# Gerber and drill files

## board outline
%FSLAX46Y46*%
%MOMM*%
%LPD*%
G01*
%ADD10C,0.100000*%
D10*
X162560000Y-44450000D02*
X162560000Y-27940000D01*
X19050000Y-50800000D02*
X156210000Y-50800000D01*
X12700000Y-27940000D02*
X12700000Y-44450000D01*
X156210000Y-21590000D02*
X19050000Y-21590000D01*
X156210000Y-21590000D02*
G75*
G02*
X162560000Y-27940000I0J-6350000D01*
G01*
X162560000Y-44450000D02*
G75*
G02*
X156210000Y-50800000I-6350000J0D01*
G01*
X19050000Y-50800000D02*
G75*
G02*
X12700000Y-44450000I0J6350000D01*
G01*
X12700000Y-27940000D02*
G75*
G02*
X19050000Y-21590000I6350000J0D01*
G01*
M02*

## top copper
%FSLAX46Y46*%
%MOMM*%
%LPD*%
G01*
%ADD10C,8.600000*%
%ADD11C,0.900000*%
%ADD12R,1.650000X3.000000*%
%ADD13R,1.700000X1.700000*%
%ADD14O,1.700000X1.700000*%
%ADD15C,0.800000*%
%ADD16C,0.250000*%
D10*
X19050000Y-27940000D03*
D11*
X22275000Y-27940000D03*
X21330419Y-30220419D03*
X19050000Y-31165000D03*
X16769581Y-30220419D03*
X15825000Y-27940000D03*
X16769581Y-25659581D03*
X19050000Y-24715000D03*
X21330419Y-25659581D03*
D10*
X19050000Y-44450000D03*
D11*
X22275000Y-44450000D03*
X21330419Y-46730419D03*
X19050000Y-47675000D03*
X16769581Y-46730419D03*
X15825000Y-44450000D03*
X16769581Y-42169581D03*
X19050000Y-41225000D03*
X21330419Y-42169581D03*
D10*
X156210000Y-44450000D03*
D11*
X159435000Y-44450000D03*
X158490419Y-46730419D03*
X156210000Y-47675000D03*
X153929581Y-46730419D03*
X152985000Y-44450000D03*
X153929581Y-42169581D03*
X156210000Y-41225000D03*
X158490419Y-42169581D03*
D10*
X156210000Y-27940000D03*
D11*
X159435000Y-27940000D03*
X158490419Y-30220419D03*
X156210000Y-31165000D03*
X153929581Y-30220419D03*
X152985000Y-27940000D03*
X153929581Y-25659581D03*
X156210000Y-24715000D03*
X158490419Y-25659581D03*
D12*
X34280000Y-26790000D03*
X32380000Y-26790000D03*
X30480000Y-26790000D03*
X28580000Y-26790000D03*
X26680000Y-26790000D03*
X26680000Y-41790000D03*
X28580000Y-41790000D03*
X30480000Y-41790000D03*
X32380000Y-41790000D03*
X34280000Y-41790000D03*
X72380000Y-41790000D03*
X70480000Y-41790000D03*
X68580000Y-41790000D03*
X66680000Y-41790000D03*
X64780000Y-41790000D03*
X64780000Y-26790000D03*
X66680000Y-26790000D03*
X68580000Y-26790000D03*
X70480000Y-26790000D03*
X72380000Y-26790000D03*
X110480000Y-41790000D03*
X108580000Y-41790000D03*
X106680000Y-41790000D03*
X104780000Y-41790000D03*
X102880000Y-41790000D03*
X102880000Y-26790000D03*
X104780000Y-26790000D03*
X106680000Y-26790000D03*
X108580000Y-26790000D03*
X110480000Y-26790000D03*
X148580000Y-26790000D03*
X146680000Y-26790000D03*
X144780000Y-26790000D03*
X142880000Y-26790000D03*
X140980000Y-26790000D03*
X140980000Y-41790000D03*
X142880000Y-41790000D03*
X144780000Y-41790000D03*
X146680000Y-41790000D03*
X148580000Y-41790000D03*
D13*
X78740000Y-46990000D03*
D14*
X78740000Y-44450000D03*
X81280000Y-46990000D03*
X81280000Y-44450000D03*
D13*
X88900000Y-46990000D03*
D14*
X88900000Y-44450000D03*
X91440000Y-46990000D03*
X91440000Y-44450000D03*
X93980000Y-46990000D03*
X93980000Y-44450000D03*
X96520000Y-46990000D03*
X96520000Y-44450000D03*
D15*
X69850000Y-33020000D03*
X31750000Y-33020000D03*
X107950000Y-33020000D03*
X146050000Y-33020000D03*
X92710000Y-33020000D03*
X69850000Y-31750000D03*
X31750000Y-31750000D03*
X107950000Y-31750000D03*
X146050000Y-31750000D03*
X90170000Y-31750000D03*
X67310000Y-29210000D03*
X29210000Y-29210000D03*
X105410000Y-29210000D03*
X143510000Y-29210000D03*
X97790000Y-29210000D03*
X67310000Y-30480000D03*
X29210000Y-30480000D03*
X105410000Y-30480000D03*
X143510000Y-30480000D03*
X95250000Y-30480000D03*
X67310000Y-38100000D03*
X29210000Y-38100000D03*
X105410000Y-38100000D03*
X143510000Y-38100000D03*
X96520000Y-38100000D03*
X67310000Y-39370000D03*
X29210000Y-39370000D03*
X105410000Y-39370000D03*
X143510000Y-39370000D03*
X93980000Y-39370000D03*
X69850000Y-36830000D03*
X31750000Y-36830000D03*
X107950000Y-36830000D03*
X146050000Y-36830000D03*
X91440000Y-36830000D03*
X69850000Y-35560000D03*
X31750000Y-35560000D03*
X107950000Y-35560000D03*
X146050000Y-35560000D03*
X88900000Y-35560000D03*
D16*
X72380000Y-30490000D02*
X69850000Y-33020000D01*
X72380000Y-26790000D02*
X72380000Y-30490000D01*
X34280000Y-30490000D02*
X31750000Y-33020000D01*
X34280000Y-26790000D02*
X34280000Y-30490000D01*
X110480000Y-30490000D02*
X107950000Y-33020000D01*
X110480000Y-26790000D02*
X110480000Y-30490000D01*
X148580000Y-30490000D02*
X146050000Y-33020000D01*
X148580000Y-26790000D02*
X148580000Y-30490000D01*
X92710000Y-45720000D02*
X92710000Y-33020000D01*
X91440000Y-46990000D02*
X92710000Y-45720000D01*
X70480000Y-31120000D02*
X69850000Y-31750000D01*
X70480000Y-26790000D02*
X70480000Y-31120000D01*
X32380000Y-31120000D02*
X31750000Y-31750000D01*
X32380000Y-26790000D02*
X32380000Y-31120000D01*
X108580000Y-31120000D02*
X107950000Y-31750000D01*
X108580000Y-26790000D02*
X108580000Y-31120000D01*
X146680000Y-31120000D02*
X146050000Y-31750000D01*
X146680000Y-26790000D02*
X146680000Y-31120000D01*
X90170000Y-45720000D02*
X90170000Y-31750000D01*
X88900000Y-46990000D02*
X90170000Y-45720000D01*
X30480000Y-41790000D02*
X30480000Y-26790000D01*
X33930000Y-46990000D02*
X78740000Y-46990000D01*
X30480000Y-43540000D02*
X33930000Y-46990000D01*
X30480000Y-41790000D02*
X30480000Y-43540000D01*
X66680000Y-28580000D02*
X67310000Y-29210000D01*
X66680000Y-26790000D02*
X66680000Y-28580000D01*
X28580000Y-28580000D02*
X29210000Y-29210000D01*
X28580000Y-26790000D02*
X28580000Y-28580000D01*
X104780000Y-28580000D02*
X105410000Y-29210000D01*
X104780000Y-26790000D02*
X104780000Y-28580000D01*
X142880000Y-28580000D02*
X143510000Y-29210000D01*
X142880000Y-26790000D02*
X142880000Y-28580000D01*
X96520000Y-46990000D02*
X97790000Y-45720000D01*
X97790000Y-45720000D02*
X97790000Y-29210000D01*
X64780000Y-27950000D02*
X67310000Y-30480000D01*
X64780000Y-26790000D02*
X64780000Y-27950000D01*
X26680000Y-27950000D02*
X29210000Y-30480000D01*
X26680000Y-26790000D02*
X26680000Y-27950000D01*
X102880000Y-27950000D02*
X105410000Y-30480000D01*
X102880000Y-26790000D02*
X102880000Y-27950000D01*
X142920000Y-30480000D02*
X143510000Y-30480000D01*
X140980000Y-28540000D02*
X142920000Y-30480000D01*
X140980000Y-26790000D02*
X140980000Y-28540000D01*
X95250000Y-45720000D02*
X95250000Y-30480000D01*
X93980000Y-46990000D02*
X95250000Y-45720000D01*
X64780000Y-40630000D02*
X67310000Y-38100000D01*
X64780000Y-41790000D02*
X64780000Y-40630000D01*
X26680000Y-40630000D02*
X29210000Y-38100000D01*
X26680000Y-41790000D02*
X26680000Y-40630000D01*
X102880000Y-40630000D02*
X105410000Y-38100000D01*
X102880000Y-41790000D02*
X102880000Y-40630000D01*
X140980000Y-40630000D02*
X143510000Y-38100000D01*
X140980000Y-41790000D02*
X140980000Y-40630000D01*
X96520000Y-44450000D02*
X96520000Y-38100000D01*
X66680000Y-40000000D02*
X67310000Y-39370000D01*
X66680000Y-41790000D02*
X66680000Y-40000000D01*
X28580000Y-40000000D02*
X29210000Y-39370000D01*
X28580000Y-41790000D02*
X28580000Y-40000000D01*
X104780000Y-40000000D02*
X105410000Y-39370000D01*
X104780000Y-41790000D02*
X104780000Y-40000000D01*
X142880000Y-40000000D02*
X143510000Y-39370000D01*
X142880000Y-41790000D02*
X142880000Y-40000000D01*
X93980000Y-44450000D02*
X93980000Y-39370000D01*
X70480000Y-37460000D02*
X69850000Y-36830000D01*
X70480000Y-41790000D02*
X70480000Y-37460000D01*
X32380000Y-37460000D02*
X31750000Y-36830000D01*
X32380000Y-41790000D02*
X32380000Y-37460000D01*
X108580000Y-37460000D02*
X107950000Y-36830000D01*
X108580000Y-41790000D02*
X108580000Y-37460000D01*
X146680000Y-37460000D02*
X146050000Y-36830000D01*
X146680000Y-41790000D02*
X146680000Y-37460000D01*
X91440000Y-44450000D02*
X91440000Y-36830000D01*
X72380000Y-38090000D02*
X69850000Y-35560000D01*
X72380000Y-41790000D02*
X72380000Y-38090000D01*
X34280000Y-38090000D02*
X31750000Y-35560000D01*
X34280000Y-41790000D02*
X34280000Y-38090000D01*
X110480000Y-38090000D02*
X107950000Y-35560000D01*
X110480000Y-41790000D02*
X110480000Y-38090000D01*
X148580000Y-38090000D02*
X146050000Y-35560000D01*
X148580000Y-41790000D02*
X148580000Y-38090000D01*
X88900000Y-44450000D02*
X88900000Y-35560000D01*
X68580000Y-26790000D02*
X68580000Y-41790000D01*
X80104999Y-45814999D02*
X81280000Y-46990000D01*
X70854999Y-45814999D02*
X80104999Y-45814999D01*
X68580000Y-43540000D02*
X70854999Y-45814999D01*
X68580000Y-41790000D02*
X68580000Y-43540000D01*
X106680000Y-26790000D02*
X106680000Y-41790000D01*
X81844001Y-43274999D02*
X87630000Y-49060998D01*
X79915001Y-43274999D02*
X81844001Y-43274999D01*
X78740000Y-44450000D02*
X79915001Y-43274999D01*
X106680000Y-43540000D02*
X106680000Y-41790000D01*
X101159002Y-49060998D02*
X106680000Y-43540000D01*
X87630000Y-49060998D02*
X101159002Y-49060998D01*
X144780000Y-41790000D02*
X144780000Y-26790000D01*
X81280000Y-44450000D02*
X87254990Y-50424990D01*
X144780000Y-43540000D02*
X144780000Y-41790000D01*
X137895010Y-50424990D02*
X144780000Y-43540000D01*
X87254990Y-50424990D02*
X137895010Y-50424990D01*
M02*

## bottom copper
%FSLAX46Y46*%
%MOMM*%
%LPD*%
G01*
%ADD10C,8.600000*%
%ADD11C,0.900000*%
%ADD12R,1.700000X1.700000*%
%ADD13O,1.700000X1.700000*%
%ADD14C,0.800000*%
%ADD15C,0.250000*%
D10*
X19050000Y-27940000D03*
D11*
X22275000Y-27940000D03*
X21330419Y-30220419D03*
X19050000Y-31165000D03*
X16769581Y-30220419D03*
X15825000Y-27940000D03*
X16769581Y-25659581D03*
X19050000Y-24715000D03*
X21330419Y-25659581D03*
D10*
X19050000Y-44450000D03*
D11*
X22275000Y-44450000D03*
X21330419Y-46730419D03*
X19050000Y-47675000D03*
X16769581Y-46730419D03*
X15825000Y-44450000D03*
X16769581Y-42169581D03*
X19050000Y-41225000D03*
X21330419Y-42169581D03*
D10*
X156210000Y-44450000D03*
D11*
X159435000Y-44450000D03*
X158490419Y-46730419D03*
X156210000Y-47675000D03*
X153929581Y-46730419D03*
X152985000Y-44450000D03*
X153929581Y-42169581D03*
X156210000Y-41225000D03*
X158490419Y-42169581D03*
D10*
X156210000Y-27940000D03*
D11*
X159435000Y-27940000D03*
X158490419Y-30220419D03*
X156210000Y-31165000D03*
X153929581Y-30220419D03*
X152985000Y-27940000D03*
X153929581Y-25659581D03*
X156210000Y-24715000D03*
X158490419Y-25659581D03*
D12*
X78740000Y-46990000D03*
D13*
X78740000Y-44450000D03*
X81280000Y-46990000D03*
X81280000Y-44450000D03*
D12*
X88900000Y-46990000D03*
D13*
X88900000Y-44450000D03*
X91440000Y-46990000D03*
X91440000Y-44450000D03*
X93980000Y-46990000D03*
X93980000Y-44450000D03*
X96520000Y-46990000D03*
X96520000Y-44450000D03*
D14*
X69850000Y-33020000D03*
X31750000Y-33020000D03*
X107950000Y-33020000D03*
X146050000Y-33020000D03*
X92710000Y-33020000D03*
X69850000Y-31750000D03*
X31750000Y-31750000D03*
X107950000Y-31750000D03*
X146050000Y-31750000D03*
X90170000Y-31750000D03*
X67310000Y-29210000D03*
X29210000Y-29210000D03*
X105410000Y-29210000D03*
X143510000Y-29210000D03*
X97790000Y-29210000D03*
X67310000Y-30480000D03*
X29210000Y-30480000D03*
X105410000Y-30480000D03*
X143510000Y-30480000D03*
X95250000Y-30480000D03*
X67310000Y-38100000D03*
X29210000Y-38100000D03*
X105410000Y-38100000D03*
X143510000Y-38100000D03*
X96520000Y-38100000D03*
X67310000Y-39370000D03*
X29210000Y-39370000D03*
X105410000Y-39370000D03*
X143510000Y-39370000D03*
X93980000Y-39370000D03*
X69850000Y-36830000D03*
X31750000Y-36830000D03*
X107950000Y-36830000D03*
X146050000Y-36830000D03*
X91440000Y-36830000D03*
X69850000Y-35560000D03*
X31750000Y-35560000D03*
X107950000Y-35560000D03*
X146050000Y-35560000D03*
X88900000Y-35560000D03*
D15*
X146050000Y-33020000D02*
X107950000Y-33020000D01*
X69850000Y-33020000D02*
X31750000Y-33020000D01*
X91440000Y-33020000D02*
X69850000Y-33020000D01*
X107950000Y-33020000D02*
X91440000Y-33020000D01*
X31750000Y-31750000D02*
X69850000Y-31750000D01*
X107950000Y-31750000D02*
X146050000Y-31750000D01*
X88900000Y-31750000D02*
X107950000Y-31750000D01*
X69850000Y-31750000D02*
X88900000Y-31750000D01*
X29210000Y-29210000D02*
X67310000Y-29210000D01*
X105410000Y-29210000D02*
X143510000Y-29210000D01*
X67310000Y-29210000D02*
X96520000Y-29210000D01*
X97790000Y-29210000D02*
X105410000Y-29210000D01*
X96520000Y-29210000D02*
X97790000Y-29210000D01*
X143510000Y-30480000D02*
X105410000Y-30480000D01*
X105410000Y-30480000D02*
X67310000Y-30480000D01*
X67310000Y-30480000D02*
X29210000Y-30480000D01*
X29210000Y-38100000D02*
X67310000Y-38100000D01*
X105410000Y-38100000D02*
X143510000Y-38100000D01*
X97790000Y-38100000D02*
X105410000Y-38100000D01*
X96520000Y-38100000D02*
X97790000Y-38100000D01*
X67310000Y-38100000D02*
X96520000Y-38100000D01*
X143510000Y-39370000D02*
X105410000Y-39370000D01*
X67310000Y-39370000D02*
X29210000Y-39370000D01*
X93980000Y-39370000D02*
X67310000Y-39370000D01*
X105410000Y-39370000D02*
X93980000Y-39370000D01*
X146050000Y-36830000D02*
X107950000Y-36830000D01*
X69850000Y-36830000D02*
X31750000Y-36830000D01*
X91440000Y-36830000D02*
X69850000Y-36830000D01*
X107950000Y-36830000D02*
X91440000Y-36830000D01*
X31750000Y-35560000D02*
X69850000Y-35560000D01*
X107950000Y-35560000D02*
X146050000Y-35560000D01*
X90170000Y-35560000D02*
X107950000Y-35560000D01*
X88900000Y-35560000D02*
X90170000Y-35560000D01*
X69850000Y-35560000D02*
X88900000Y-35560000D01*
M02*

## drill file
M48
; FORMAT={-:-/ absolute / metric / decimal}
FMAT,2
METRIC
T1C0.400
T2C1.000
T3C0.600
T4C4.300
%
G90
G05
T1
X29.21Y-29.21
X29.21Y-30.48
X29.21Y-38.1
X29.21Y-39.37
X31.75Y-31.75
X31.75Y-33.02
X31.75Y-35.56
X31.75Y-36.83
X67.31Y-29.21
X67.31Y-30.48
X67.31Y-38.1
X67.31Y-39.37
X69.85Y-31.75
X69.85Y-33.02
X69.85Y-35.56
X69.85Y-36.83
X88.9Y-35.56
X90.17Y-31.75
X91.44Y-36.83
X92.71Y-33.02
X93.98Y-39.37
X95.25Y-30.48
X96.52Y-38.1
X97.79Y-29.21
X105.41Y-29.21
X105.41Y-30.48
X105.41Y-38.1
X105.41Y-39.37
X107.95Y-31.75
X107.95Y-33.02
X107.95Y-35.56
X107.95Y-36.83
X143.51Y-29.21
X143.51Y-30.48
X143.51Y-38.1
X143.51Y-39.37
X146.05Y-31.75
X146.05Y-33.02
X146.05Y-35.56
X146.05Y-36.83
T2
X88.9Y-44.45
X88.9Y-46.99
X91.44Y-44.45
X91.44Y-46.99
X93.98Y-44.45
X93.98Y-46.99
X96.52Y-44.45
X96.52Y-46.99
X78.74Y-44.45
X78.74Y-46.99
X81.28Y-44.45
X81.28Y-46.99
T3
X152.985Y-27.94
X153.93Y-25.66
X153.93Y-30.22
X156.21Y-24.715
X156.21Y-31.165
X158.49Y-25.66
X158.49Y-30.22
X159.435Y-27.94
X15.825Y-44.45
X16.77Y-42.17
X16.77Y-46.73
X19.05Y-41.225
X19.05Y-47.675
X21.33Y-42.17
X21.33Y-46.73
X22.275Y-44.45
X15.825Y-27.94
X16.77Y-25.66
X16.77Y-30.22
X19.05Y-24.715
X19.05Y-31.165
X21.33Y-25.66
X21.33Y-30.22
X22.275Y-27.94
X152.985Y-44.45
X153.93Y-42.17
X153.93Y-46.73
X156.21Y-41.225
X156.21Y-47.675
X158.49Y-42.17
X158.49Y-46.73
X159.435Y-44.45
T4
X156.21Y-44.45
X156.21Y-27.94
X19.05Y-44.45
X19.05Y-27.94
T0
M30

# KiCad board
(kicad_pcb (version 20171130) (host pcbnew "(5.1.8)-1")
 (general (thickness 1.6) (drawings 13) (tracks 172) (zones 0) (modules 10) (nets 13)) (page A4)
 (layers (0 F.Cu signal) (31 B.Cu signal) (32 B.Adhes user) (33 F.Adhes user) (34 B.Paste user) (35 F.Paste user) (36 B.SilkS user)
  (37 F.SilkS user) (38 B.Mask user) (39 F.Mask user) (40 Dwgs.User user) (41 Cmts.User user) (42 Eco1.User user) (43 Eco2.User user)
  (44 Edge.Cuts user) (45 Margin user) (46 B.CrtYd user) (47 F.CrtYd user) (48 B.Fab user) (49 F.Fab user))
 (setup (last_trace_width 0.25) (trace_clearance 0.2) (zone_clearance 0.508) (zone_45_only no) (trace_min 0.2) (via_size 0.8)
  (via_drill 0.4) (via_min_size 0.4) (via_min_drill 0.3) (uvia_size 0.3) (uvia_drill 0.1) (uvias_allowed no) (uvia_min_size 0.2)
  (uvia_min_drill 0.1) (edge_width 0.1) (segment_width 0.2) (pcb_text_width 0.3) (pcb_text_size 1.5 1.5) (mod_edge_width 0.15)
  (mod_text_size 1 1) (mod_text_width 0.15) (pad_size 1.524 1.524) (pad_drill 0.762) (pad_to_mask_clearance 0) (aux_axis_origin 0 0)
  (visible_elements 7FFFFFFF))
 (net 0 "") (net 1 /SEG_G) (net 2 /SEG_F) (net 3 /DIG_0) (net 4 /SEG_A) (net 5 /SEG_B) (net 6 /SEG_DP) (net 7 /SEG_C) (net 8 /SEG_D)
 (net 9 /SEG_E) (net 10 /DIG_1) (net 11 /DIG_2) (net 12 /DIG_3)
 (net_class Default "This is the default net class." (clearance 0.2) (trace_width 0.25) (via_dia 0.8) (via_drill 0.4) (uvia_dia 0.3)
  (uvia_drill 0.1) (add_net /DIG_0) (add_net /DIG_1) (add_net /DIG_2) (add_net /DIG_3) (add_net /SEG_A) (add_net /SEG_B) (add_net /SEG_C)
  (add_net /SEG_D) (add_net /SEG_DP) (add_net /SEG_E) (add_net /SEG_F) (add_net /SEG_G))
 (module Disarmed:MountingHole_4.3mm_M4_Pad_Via (layer F.Cu) (at 19.05 27.94)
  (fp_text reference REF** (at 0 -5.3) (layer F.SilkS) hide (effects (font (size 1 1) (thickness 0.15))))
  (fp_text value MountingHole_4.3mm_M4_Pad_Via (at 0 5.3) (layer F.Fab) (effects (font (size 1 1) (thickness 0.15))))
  (pad "" np_thru_hole circle (at 0 0) (size 8.6 8.6) (drill 4.3) (layers *.Cu *.Mask))
  (pad "" np_thru_hole circle (at 3.225 0) (size 0.9 0.9) (drill 0.6) (layers *.Cu *.Mask))
  (pad "" np_thru_hole circle (at 2.280419 2.280419) (size 0.9 0.9) (drill 0.6) (layers *.Cu *.Mask))
  (pad "" np_thru_hole circle (at 0 3.225) (size 0.9 0.9) (drill 0.6) (layers *.Cu *.Mask))
  (pad "" np_thru_hole circle (at -2.280419 2.280419) (size 0.9 0.9) (drill 0.6) (layers *.Cu *.Mask))
  (pad "" np_thru_hole circle (at -3.225 0) (size 0.9 0.9) (drill 0.6) (layers *.Cu *.Mask))
  (pad "" np_thru_hole circle (at -2.280419 -2.280419) (size 0.9 0.9) (drill 0.6) (layers *.Cu *.Mask))
  (pad "" np_thru_hole circle (at 0 -3.225) (size 0.9 0.9) (drill 0.6) (layers *.Cu *.Mask))
  (pad "" np_thru_hole circle (at 2.280419 -2.280419) (size 0.9 0.9) (drill 0.6) (layers *.Cu *.Mask)))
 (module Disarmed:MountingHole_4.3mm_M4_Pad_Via (layer F.Cu) (at 19.05 44.45)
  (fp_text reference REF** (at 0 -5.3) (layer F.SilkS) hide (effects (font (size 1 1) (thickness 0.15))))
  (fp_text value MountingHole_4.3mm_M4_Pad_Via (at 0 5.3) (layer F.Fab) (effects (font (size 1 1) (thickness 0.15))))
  (pad "" np_thru_hole circle (at 0 0) (size 8.6 8.6) (drill 4.3) (layers *.Cu *.Mask))
  (pad "" np_thru_hole circle (at 3.225 0) (size 0.9 0.9) (drill 0.6) (layers *.Cu *.Mask))
  (pad "" np_thru_hole circle (at 2.280419 2.280419) (size 0.9 0.9) (drill 0.6) (layers *.Cu *.Mask))
  (pad "" np_thru_hole circle (at 0 3.225) (size 0.9 0.9) (drill 0.6) (layers *.Cu *.Mask))
  (pad "" np_thru_hole circle (at -2.280419 2.280419) (size 0.9 0.9) (drill 0.6) (layers *.Cu *.Mask))
  (pad "" np_thru_hole circle (at -3.225 0) (size 0.9 0.9) (drill 0.6) (layers *.Cu *.Mask))
  (pad "" np_thru_hole circle (at -2.280419 -2.280419) (size 0.9 0.9) (drill 0.6) (layers *.Cu *.Mask))
  (pad "" np_thru_hole circle (at 0 -3.225) (size 0.9 0.9) (drill 0.6) (layers *.Cu *.Mask))
  (pad "" np_thru_hole circle (at 2.280419 -2.280419) (size 0.9 0.9) (drill 0.6) (layers *.Cu *.Mask)))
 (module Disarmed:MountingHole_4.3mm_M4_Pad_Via (layer F.Cu) (at 156.21 44.45)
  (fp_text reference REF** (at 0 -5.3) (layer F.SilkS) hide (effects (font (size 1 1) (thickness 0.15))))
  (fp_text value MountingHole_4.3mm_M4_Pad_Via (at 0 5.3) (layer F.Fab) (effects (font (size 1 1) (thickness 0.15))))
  (pad "" np_thru_hole circle (at 0 0) (size 8.6 8.6) (drill 4.3) (layers *.Cu *.Mask))
  (pad "" np_thru_hole circle (at 3.225 0) (size 0.9 0.9) (drill 0.6) (layers *.Cu *.Mask))
  (pad "" np_thru_hole circle (at 2.280419 2.280419) (size 0.9 0.9) (drill 0.6) (layers *.Cu *.Mask))
  (pad "" np_thru_hole circle (at 0 3.225) (size 0.9 0.9) (drill 0.6) (layers *.Cu *.Mask))
  (pad "" np_thru_hole circle (at -2.280419 2.280419) (size 0.9 0.9) (drill 0.6) (layers *.Cu *.Mask))
  (pad "" np_thru_hole circle (at -3.225 0) (size 0.9 0.9) (drill 0.6) (layers *.Cu *.Mask))
  (pad "" np_thru_hole circle (at -2.280419 -2.280419) (size 0.9 0.9) (drill 0.6) (layers *.Cu *.Mask))
  (pad "" np_thru_hole circle (at 0 -3.225) (size 0.9 0.9) (drill 0.6) (layers *.Cu *.Mask))
  (pad "" np_thru_hole circle (at 2.280419 -2.280419) (size 0.9 0.9) (drill 0.6) (layers *.Cu *.Mask)))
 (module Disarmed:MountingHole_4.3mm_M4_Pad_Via (layer F.Cu) (at 156.21 27.94)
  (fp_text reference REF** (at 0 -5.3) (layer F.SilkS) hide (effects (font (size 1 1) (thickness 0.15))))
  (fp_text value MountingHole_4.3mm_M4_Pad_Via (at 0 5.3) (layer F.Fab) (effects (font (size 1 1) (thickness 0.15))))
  (pad "" np_thru_hole circle (at 0 0) (size 8.6 8.6) (drill 4.3) (layers *.Cu *.Mask))
  (pad "" np_thru_hole circle (at 3.225 0) (size 0.9 0.9) (drill 0.6) (layers *.Cu *.Mask))
  (pad "" np_thru_hole circle (at 2.280419 2.280419) (size 0.9 0.9) (drill 0.6) (layers *.Cu *.Mask))
  (pad "" np_thru_hole circle (at 0 3.225) (size 0.9 0.9) (drill 0.6) (layers *.Cu *.Mask))
  (pad "" np_thru_hole circle (at -2.280419 2.280419) (size 0.9 0.9) (drill 0.6) (layers *.Cu *.Mask))
  (pad "" np_thru_hole circle (at -3.225 0) (size 0.9 0.9) (drill 0.6) (layers *.Cu *.Mask))
  (pad "" np_thru_hole circle (at -2.280419 -2.280419) (size 0.9 0.9) (drill 0.6) (layers *.Cu *.Mask))
  (pad "" np_thru_hole circle (at 0 -3.225) (size 0.9 0.9) (drill 0.6) (layers *.Cu *.Mask))
  (pad "" np_thru_hole circle (at 2.280419 -2.280419) (size 0.9 0.9) (drill 0.6) (layers *.Cu *.Mask)))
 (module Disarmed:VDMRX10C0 (layer F.Cu) (at 30.48 34.29)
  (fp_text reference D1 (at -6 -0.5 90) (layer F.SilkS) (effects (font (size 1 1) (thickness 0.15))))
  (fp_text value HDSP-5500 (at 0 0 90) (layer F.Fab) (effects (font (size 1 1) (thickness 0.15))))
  (pad 10 smd rect (at 3.8 -7.5) (size 1.65 3) (layers F.Cu F.Paste F.Mask) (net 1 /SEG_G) (clearance 0.2875))
  (pad 9 smd rect (at 1.9 -7.5) (size 1.65 3) (layers F.Cu F.Paste F.Mask) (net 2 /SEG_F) (clearance 0.2875))
  (pad 8 smd rect (at 0 -7.5) (size 1.65 3) (layers F.Cu F.Paste F.Mask) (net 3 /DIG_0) (clearance 0.2875))
  (pad 7 smd rect (at -1.9 -7.5) (size 1.65 3) (layers F.Cu F.Paste F.Mask) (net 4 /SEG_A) (clearance 0.2875))
  (pad 6 smd rect (at -3.8 -7.5) (size 1.65 3) (layers F.Cu F.Paste F.Mask) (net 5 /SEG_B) (clearance 0.2875))
  (pad 5 smd rect (at -3.8 7.5) (size 1.65 3) (layers F.Cu F.Paste F.Mask) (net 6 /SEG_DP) (clearance 0.2875))
  (pad 4 smd rect (at -1.9 7.5) (size 1.65 3) (layers F.Cu F.Paste F.Mask) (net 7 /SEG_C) (clearance 0.2875))
  (pad 3 smd rect (at 0 7.5) (size 1.65 3) (layers F.Cu F.Paste F.Mask) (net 3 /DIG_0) (clearance 0.2875))
  (pad 2 smd rect (at 1.9 7.5) (size 1.65 3) (layers F.Cu F.Paste F.Mask) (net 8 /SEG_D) (clearance 0.2875))
  (pad 1 smd rect (at 3.8 7.5) (size 1.65 3) (layers F.Cu F.Paste F.Mask) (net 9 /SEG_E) (clearance 0.2875)))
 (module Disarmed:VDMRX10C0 (layer F.Cu) (at 68.58 34.29)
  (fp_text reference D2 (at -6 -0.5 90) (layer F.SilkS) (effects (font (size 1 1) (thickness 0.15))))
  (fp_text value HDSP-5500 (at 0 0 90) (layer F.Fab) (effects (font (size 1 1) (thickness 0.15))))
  (pad 1 smd rect (at 3.8 7.5) (size 1.65 3) (layers F.Cu F.Paste F.Mask) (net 9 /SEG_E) (clearance 0.2875))
  (pad 2 smd rect (at 1.9 7.5) (size 1.65 3) (layers F.Cu F.Paste F.Mask) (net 8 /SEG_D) (clearance 0.2875))
  (pad 3 smd rect (at 0 7.5) (size 1.65 3) (layers F.Cu F.Paste F.Mask) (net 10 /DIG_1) (clearance 0.2875))
  (pad 4 smd rect (at -1.9 7.5) (size 1.65 3) (layers F.Cu F.Paste F.Mask) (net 7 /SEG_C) (clearance 0.2875))
  (pad 5 smd rect (at -3.8 7.5) (size 1.65 3) (layers F.Cu F.Paste F.Mask) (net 6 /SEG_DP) (clearance 0.2875))
  (pad 6 smd rect (at -3.8 -7.5) (size 1.65 3) (layers F.Cu F.Paste F.Mask) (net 5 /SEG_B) (clearance 0.2875))
  (pad 7 smd rect (at -1.9 -7.5) (size 1.65 3) (layers F.Cu F.Paste F.Mask) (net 4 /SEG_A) (clearance 0.2875))
  (pad 8 smd rect (at 0 -7.5) (size 1.65 3) (layers F.Cu F.Paste F.Mask) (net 10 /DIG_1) (clearance 0.2875))
  (pad 9 smd rect (at 1.9 -7.5) (size 1.65 3) (layers F.Cu F.Paste F.Mask) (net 2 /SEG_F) (clearance 0.2875))
  (pad 10 smd rect (at 3.8 -7.5) (size 1.65 3) (layers F.Cu F.Paste F.Mask) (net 1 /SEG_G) (clearance 0.2875)))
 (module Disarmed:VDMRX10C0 (layer F.Cu) (at 106.68 34.29)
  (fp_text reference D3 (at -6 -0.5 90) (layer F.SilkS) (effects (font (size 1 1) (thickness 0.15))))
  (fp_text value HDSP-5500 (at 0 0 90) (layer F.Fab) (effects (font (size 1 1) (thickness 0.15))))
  (pad 1 smd rect (at 3.8 7.5) (size 1.65 3) (layers F.Cu F.Paste F.Mask) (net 9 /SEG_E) (clearance 0.2875))
  (pad 2 smd rect (at 1.9 7.5) (size 1.65 3) (layers F.Cu F.Paste F.Mask) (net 8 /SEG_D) (clearance 0.2875))
  (pad 3 smd rect (at 0 7.5) (size 1.65 3) (layers F.Cu F.Paste F.Mask) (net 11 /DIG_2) (clearance 0.2875))
  (pad 4 smd rect (at -1.9 7.5) (size 1.65 3) (layers F.Cu F.Paste F.Mask) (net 7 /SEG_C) (clearance 0.2875))
  (pad 5 smd rect (at -3.8 7.5) (size 1.65 3) (layers F.Cu F.Paste F.Mask) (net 6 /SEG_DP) (clearance 0.2875))
  (pad 6 smd rect (at -3.8 -7.5) (size 1.65 3) (layers F.Cu F.Paste F.Mask) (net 5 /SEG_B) (clearance 0.2875))
  (pad 7 smd rect (at -1.9 -7.5) (size 1.65 3) (layers F.Cu F.Paste F.Mask) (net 4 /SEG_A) (clearance 0.2875))
  (pad 8 smd rect (at 0 -7.5) (size 1.65 3) (layers F.Cu F.Paste F.Mask) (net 11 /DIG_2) (clearance 0.2875))
  (pad 9 smd rect (at 1.9 -7.5) (size 1.65 3) (layers F.Cu F.Paste F.Mask) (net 2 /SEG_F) (clearance 0.2875))
  (pad 10 smd rect (at 3.8 -7.5) (size 1.65 3) (layers F.Cu F.Paste F.Mask) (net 1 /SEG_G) (clearance 0.2875)))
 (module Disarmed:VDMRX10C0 (layer F.Cu) (at 144.78 34.29)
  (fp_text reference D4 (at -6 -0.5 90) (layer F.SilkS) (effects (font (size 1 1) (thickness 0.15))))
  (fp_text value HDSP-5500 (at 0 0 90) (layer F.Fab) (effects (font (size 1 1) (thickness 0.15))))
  (pad 10 smd rect (at 3.8 -7.5) (size 1.65 3) (layers F.Cu F.Paste F.Mask) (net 1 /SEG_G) (clearance 0.2875))
  (pad 9 smd rect (at 1.9 -7.5) (size 1.65 3) (layers F.Cu F.Paste F.Mask) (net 2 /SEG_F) (clearance 0.2875))
  (pad 8 smd rect (at 0 -7.5) (size 1.65 3) (layers F.Cu F.Paste F.Mask) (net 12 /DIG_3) (clearance 0.2875))
  (pad 7 smd rect (at -1.9 -7.5) (size 1.65 3) (layers F.Cu F.Paste F.Mask) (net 4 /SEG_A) (clearance 0.2875))
  (pad 6 smd rect (at -3.8 -7.5) (size 1.65 3) (layers F.Cu F.Paste F.Mask) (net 5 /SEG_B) (clearance 0.2875))
  (pad 5 smd rect (at -3.8 7.5) (size 1.65 3) (layers F.Cu F.Paste F.Mask) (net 6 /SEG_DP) (clearance 0.2875))
  (pad 4 smd rect (at -1.9 7.5) (size 1.65 3) (layers F.Cu F.Paste F.Mask) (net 7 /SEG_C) (clearance 0.2875))
  (pad 3 smd rect (at 0 7.5) (size 1.65 3) (layers F.Cu F.Paste F.Mask) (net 12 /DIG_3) (clearance 0.2875))
  (pad 2 smd rect (at 1.9 7.5) (size 1.65 3) (layers F.Cu F.Paste F.Mask) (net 8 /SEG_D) (clearance 0.2875))
  (pad 1 smd rect (at 3.8 7.5) (size 1.65 3) (layers F.Cu F.Paste F.Mask) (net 9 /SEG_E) (clearance 0.2875)))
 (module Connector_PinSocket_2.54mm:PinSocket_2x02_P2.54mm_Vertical (layer B.Cu) (at 78.74 46.99 270)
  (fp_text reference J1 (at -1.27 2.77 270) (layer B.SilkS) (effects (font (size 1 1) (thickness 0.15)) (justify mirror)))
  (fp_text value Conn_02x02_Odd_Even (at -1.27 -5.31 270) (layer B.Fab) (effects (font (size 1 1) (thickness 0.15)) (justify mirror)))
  (pad 1 thru_hole rect (at 0 0 270) (size 1.7 1.7) (drill 1) (layers *.Cu *.Mask) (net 3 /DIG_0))
  (pad 2 thru_hole oval (at -2.54 0 270) (size 1.7 1.7) (drill 1) (layers *.Cu *.Mask) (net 11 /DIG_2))
  (pad 3 thru_hole oval (at 0 -2.54 270) (size 1.7 1.7) (drill 1) (layers *.Cu *.Mask) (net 10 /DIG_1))
  (pad 4 thru_hole oval (at -2.54 -2.54 270) (size 1.7 1.7) (drill 1) (layers *.Cu *.Mask) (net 12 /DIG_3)))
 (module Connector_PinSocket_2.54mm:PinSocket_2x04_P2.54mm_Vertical (layer B.Cu) (at 88.9 46.99 270)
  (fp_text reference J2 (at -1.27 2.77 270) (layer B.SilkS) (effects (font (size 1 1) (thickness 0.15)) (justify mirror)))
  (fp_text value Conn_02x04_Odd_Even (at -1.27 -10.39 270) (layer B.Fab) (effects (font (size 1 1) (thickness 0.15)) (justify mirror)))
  (pad 1 thru_hole rect (at 0 0 270) (size 1.7 1.7) (drill 1) (layers *.Cu *.Mask) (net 2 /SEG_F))
  (pad 2 thru_hole oval (at -2.54 0 270) (size 1.7 1.7) (drill 1) (layers *.Cu *.Mask) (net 9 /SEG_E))
  (pad 3 thru_hole oval (at 0 -2.54 270) (size 1.7 1.7) (drill 1) (layers *.Cu *.Mask) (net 1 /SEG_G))
  (pad 4 thru_hole oval (at -2.54 -2.54 270) (size 1.7 1.7) (drill 1) (layers *.Cu *.Mask) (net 8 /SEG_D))
  (pad 5 thru_hole oval (at 0 -5.08 270) (size 1.7 1.7) (drill 1) (layers *.Cu *.Mask) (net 5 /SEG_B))
  (pad 6 thru_hole oval (at -2.54 -5.08 270) (size 1.7 1.7) (drill 1) (layers *.Cu *.Mask) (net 7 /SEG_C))
  (pad 7 thru_hole oval (at 0 -7.62 270) (size 1.7 1.7) (drill 1) (layers *.Cu *.Mask) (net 4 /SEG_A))
  (pad 8 thru_hole oval (at -2.54 -7.62 270) (size 1.7 1.7) (drill 1) (layers *.Cu *.Mask) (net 6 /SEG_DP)))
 (gr_line (start 162.56 44.45) (end 162.56 27.94) (layer Edge.Cuts) (width 0.1))
 (gr_line (start 19.05 50.8) (end 156.21 50.8) (layer Edge.Cuts) (width 0.1))
 (gr_line (start 12.7 27.94) (end 12.7 44.45) (layer Edge.Cuts) (width 0.1))
 (gr_line (start 156.21 21.59) (end 19.05 21.59) (layer Edge.Cuts) (width 0.1))
 (gr_arc (start 156.21 27.94) (end 162.56 27.94) (angle -90) (layer Edge.Cuts) (width 0.1))
 (gr_arc (start 156.21 44.45) (end 156.21 50.8) (angle -90) (layer Edge.Cuts) (width 0.1))
 (gr_arc (start 19.05 44.45) (end 12.7 44.45) (angle -90) (layer Edge.Cuts) (width 0.1))
 (gr_arc (start 19.05 27.94) (end 19.05 21.59) (angle -90) (layer Edge.Cuts) (width 0.1))
 (via (at 69.85 33.02) (size 0.8) (drill 0.4) (layers F.Cu B.Cu) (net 1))
 (segment (start 72.38 30.49) (end 69.85 33.02) (width 0.25) (layer F.Cu) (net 1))
 (segment (start 72.38 26.79) (end 72.38 30.49) (width 0.25) (layer F.Cu) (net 1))
 (via (at 31.75 33.02) (size 0.8) (drill 0.4) (layers F.Cu B.Cu) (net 1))
 (segment (start 34.28 30.49) (end 31.75 33.02) (width 0.25) (layer F.Cu) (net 1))
 (segment (start 34.28 26.79) (end 34.28 30.49) (width 0.25) (layer F.Cu) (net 1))
 (via (at 107.95 33.02) (size 0.8) (drill 0.4) (layers F.Cu B.Cu) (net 1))
 (segment (start 110.48 30.49) (end 107.95 33.02) (width 0.25) (layer F.Cu) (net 1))
 (segment (start 110.48 26.79) (end 110.48 30.49) (width 0.25) (layer F.Cu) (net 1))
 (via (at 146.05 33.02) (size 0.8) (drill 0.4) (layers F.Cu B.Cu) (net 1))
 (segment (start 148.58 30.49) (end 146.05 33.02) (width 0.25) (layer F.Cu) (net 1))
 (segment (start 148.58 26.79) (end 148.58 30.49) (width 0.25) (layer F.Cu) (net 1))
 (segment (start 146.05 33.02) (end 107.95 33.02) (width 0.25) (layer B.Cu) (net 1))
 (segment (start 69.85 33.02) (end 31.75 33.02) (width 0.25) (layer B.Cu) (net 1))
 (segment (start 91.44 33.02) (end 69.85 33.02) (width 0.25) (layer B.Cu) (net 1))
 (segment (start 107.95 33.02) (end 91.44 33.02) (width 0.25) (layer B.Cu) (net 1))
 (segment (start 92.71 45.72) (end 92.71 33.02) (width 0.25) (layer F.Cu) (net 1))
 (via (at 92.71 33.02) (size 0.8) (drill 0.4) (layers F.Cu B.Cu) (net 1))
 (segment (start 91.44 46.99) (end 92.71 45.72) (width 0.25) (layer F.Cu) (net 1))
 (via (at 69.85 31.75) (size 0.8) (drill 0.4) (layers F.Cu B.Cu) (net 2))
 (segment (start 70.48 31.12) (end 69.85 31.75) (width 0.25) (layer F.Cu) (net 2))
 (segment (start 70.48 26.79) (end 70.48 31.12) (width 0.25) (layer F.Cu) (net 2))
 (via (at 31.75 31.75) (size 0.8) (drill 0.4) (layers F.Cu B.Cu) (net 2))
 (segment (start 32.38 31.12) (end 31.75 31.75) (width 0.25) (layer F.Cu) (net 2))
 (segment (start 32.38 26.79) (end 32.38 31.12) (width 0.25) (layer F.Cu) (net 2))
 (via (at 107.95 31.75) (size 0.8) (drill 0.4) (layers F.Cu B.Cu) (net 2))
 (segment (start 108.58 31.12) (end 107.95 31.75) (width 0.25) (layer F.Cu) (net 2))
 (segment (start 108.58 26.79) (end 108.58 31.12) (width 0.25) (layer F.Cu) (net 2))
 (via (at 146.05 31.75) (size 0.8) (drill 0.4) (layers F.Cu B.Cu) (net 2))
 (segment (start 146.68 31.12) (end 146.05 31.75) (width 0.25) (layer F.Cu) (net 2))
 (segment (start 146.68 26.79) (end 146.68 31.12) (width 0.25) (layer F.Cu) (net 2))
 (segment (start 31.75 31.75) (end 69.85 31.75) (width 0.25) (layer B.Cu) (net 2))
 (segment (start 107.95 31.75) (end 146.05 31.75) (width 0.25) (layer B.Cu) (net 2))
 (segment (start 88.9 31.75) (end 107.95 31.75) (width 0.25) (layer B.Cu) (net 2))
 (segment (start 69.85 31.75) (end 88.9 31.75) (width 0.25) (layer B.Cu) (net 2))
 (via (at 90.17 31.75) (size 0.8) (drill 0.4) (layers F.Cu B.Cu) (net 2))
 (segment (start 90.17 45.72) (end 90.17 31.75) (width 0.25) (layer F.Cu) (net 2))
 (segment (start 88.9 46.99) (end 90.17 45.72) (width 0.25) (layer F.Cu) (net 2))
 (segment (start 30.48 41.79) (end 30.48 26.79) (width 0.25) (layer F.Cu) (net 3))
 (segment (start 33.93 46.99) (end 78.74 46.99) (width 0.25) (layer F.Cu) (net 3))
 (segment (start 30.48 43.54) (end 33.93 46.99) (width 0.25) (layer F.Cu) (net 3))
 (segment (start 30.48 41.79) (end 30.48 43.54) (width 0.25) (layer F.Cu) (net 3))
 (via (at 67.31 29.21) (size 0.8) (drill 0.4) (layers F.Cu B.Cu) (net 4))
 (segment (start 66.68 28.58) (end 67.31 29.21) (width 0.25) (layer F.Cu) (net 4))
 (segment (start 66.68 26.79) (end 66.68 28.58) (width 0.25) (layer F.Cu) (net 4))
 (via (at 29.21 29.21) (size 0.8) (drill 0.4) (layers F.Cu B.Cu) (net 4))
 (segment (start 28.58 28.58) (end 29.21 29.21) (width 0.25) (layer F.Cu) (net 4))
 (segment (start 28.58 26.79) (end 28.58 28.58) (width 0.25) (layer F.Cu) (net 4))
 (via (at 105.41 29.21) (size 0.8) (drill 0.4) (layers F.Cu B.Cu) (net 4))
 (segment (start 104.78 28.58) (end 105.41 29.21) (width 0.25) (layer F.Cu) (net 4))
 (segment (start 104.78 26.79) (end 104.78 28.58) (width 0.25) (layer F.Cu) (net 4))
 (segment (start 142.88 28.58) (end 143.51 29.21) (width 0.25) (layer F.Cu) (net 4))
 (via (at 143.51 29.21) (size 0.8) (drill 0.4) (layers F.Cu B.Cu) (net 4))
 (segment (start 142.88 26.79) (end 142.88 28.58) (width 0.25) (layer F.Cu) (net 4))
 (segment (start 29.21 29.21) (end 67.31 29.21) (width 0.25) (layer B.Cu) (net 4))
 (segment (start 105.41 29.21) (end 143.51 29.21) (width 0.25) (layer B.Cu) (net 4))
 (segment (start 67.31 29.21) (end 96.52 29.21) (width 0.25) (layer B.Cu) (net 4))
 (via (at 97.79 29.21) (size 0.8) (drill 0.4) (layers F.Cu B.Cu) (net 4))
 (segment (start 96.52 46.99) (end 97.79 45.72) (width 0.25) (layer F.Cu) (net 4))
 (segment (start 97.79 29.21) (end 105.41 29.21) (width 0.25) (layer B.Cu) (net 4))
 (segment (start 97.79 45.72) (end 97.79 29.21) (width 0.25) (layer F.Cu) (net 4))
 (segment (start 96.52 29.21) (end 97.79 29.21) (width 0.25) (layer B.Cu) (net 4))
 (via (at 67.31 30.48) (size 0.8) (drill 0.4) (layers F.Cu B.Cu) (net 5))
 (segment (start 64.78 27.95) (end 67.31 30.48) (width 0.25) (layer F.Cu) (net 5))
 (segment (start 64.78 26.79) (end 64.78 27.95) (width 0.25) (layer F.Cu) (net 5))
 (via (at 29.21 30.48) (size 0.8) (drill 0.4) (layers F.Cu B.Cu) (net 5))
 (segment (start 26.68 27.95) (end 29.21 30.48) (width 0.25) (layer F.Cu) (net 5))
 (segment (start 26.68 26.79) (end 26.68 27.95) (width 0.25) (layer F.Cu) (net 5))
 (via (at 105.41 30.48) (size 0.8) (drill 0.4) (layers F.Cu B.Cu) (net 5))
 (segment (start 102.88 27.95) (end 105.41 30.48) (width 0.25) (layer F.Cu) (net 5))
 (segment (start 102.88 26.79) (end 102.88 27.95) (width 0.25) (layer F.Cu) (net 5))
 (via (at 143.51 30.48) (size 0.8) (drill 0.4) (layers F.Cu B.Cu) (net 5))
 (segment (start 142.92 30.48) (end 143.51 30.48) (width 0.25) (layer F.Cu) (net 5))
 (segment (start 140.98 28.54) (end 142.92 30.48) (width 0.25) (layer F.Cu) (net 5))
 (segment (start 140.98 26.79) (end 140.98 28.54) (width 0.25) (layer F.Cu) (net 5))
 (segment (start 143.51 30.48) (end 105.41 30.48) (width 0.25) (layer B.Cu) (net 5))
 (segment (start 105.41 30.48) (end 67.31 30.48) (width 0.25) (layer B.Cu) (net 5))
 (segment (start 67.31 30.48) (end 29.21 30.48) (width 0.25) (layer B.Cu) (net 5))
 (segment (start 95.25 45.72) (end 95.25 30.48) (width 0.25) (layer F.Cu) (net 5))
 (via (at 95.25 30.48) (size 0.8) (drill 0.4) (layers F.Cu B.Cu) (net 5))
 (segment (start 93.98 46.99) (end 95.25 45.72) (width 0.25) (layer F.Cu) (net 5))
 (via (at 67.31 38.1) (size 0.8) (drill 0.4) (layers F.Cu B.Cu) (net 6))
 (segment (start 64.78 40.63) (end 67.31 38.1) (width 0.25) (layer F.Cu) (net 6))
 (segment (start 64.78 41.79) (end 64.78 40.63) (width 0.25) (layer F.Cu) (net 6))
 (via (at 29.21 38.1) (size 0.8) (drill 0.4) (layers F.Cu B.Cu) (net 6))
 (segment (start 26.68 40.63) (end 29.21 38.1) (width 0.25) (layer F.Cu) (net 6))
 (segment (start 26.68 41.79) (end 26.68 40.63) (width 0.25) (layer F.Cu) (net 6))
 (via (at 105.41 38.1) (size 0.8) (drill 0.4) (layers F.Cu B.Cu) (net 6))
 (segment (start 102.88 40.63) (end 105.41 38.1) (width 0.25) (layer F.Cu) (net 6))
 (segment (start 102.88 41.79) (end 102.88 40.63) (width 0.25) (layer F.Cu) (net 6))
 (via (at 143.51 38.1) (size 0.8) (drill 0.4) (layers F.Cu B.Cu) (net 6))
 (segment (start 140.98 40.63) (end 143.51 38.1) (width 0.25) (layer F.Cu) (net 6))
 (segment (start 140.98 41.79) (end 140.98 40.63) (width 0.25) (layer F.Cu) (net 6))
 (segment (start 29.21 38.1) (end 67.31 38.1) (width 0.25) (layer B.Cu) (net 6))
 (segment (start 105.41 38.1) (end 143.51 38.1) (width 0.25) (layer B.Cu) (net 6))
 (segment (start 97.79 38.1) (end 105.41 38.1) (width 0.25) (layer B.Cu) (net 6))
 (via (at 96.52 38.1) (size 0.8) (drill 0.4) (layers F.Cu B.Cu) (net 6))
 (segment (start 96.52 44.45) (end 96.52 38.1) (width 0.25) (layer F.Cu) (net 6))
 (segment (start 96.52 38.1) (end 97.79 38.1) (width 0.25) (layer B.Cu) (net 6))
 (segment (start 67.31 38.1) (end 96.52 38.1) (width 0.25) (layer B.Cu) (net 6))
 (via (at 67.31 39.37) (size 0.8) (drill 0.4) (layers F.Cu B.Cu) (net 7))
 (segment (start 66.68 40) (end 67.31 39.37) (width 0.25) (layer F.Cu) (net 7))
 (segment (start 66.68 41.79) (end 66.68 40) (width 0.25) (layer F.Cu) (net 7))
 (via (at 29.21 39.37) (size 0.8) (drill 0.4) (layers F.Cu B.Cu) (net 7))
 (segment (start 28.58 40) (end 29.21 39.37) (width 0.25) (layer F.Cu) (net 7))
 (segment (start 28.58 41.79) (end 28.58 40) (width 0.25) (layer F.Cu) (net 7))
 (via (at 105.41 39.37) (size 0.8) (drill 0.4) (layers F.Cu B.Cu) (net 7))
 (segment (start 104.78 40) (end 105.41 39.37) (width 0.25) (layer F.Cu) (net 7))
 (segment (start 104.78 41.79) (end 104.78 40) (width 0.25) (layer F.Cu) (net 7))
 (via (at 143.51 39.37) (size 0.8) (drill 0.4) (layers F.Cu B.Cu) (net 7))
 (segment (start 142.88 40) (end 143.51 39.37) (width 0.25) (layer F.Cu) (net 7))
 (segment (start 142.88 41.79) (end 142.88 40) (width 0.25) (layer F.Cu) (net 7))
 (segment (start 143.51 39.37) (end 105.41 39.37) (width 0.25) (layer B.Cu) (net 7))
 (segment (start 67.31 39.37) (end 29.21 39.37) (width 0.25) (layer B.Cu) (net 7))
 (via (at 93.98 39.37) (size 0.8) (drill 0.4) (layers F.Cu B.Cu) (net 7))
 (segment (start 93.98 44.45) (end 93.98 39.37) (width 0.25) (layer F.Cu) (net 7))
 (segment (start 93.98 39.37) (end 67.31 39.37) (width 0.25) (layer B.Cu) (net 7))
 (segment (start 105.41 39.37) (end 93.98 39.37) (width 0.25) (layer B.Cu) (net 7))
 (via (at 69.85 36.83) (size 0.8) (drill 0.4) (layers F.Cu B.Cu) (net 8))
 (segment (start 70.48 37.46) (end 69.85 36.83) (width 0.25) (layer F.Cu) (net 8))
 (segment (start 70.48 41.79) (end 70.48 37.46) (width 0.25) (layer F.Cu) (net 8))
 (via (at 31.75 36.83) (size 0.8) (drill 0.4) (layers F.Cu B.Cu) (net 8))
 (segment (start 32.38 37.46) (end 31.75 36.83) (width 0.25) (layer F.Cu) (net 8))
 (segment (start 32.38 41.79) (end 32.38 37.46) (width 0.25) (layer F.Cu) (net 8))
 (via (at 107.95 36.83) (size 0.8) (drill 0.4) (layers F.Cu B.Cu) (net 8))
 (segment (start 108.58 37.46) (end 107.95 36.83) (width 0.25) (layer F.Cu) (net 8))
 (segment (start 108.58 41.79) (end 108.58 37.46) (width 0.25) (layer F.Cu) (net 8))
 (via (at 146.05 36.83) (size 0.8) (drill 0.4) (layers F.Cu B.Cu) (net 8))
 (segment (start 146.68 37.46) (end 146.05 36.83) (width 0.25) (layer F.Cu) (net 8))
 (segment (start 146.68 41.79) (end 146.68 37.46) (width 0.25) (layer F.Cu) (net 8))
 (segment (start 146.05 36.83) (end 107.95 36.83) (width 0.25) (layer B.Cu) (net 8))
 (segment (start 69.85 36.83) (end 31.75 36.83) (width 0.25) (layer B.Cu) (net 8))
 (via (at 91.44 36.83) (size 0.8) (drill 0.4) (layers F.Cu B.Cu) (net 8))
 (segment (start 91.44 44.45) (end 91.44 36.83) (width 0.25) (layer F.Cu) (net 8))
 (segment (start 91.44 36.83) (end 69.85 36.83) (width 0.25) (layer B.Cu) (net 8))
 (segment (start 107.95 36.83) (end 91.44 36.83) (width 0.25) (layer B.Cu) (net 8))
 (via (at 69.85 35.56) (size 0.8) (drill 0.4) (layers F.Cu B.Cu) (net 9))
 (segment (start 72.38 38.09) (end 69.85 35.56) (width 0.25) (layer F.Cu) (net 9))
 (segment (start 72.38 41.79) (end 72.38 38.09) (width 0.25) (layer F.Cu) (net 9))
 (via (at 31.75 35.56) (size 0.8) (drill 0.4) (layers F.Cu B.Cu) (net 9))
 (segment (start 34.28 38.09) (end 31.75 35.56) (width 0.25) (layer F.Cu) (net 9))
 (segment (start 34.28 41.79) (end 34.28 38.09) (width 0.25) (layer F.Cu) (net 9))
 (via (at 107.95 35.56) (size 0.8) (drill 0.4) (layers F.Cu B.Cu) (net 9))
 (segment (start 110.48 38.09) (end 107.95 35.56) (width 0.25) (layer F.Cu) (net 9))
 (segment (start 110.48 41.79) (end 110.48 38.09) (width 0.25) (layer F.Cu) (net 9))
 (via (at 146.05 35.56) (size 0.8) (drill 0.4) (layers F.Cu B.Cu) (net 9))
 (segment (start 148.58 38.09) (end 146.05 35.56) (width 0.25) (layer F.Cu) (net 9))
 (segment (start 148.58 41.79) (end 148.58 38.09) (width 0.25) (layer F.Cu) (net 9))
 (segment (start 31.75 35.56) (end 69.85 35.56) (width 0.25) (layer B.Cu) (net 9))
 (segment (start 107.95 35.56) (end 146.05 35.56) (width 0.25) (layer B.Cu) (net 9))
 (segment (start 90.17 35.56) (end 107.95 35.56) (width 0.25) (layer B.Cu) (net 9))
 (via (at 88.9 35.56) (size 0.8) (drill 0.4) (layers F.Cu B.Cu) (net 9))
 (segment (start 88.9 44.45) (end 88.9 35.56) (width 0.25) (layer F.Cu) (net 9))
 (segment (start 88.9 35.56) (end 90.17 35.56) (width 0.25) (layer B.Cu) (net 9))
 (segment (start 69.85 35.56) (end 88.9 35.56) (width 0.25) (layer B.Cu) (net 9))
 (segment (start 68.58 26.79) (end 68.58 41.79) (width 0.25) (layer F.Cu) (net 10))
 (segment (start 80.104999 45.814999) (end 81.28 46.99) (width 0.25) (layer F.Cu) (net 10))
 (segment (start 70.854999 45.814999) (end 80.104999 45.814999) (width 0.25) (layer F.Cu) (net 10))
 (segment (start 68.58 43.54) (end 70.854999 45.814999) (width 0.25) (layer F.Cu) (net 10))
 (segment (start 68.58 41.79) (end 68.58 43.54) (width 0.25) (layer F.Cu) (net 10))
 (segment (start 106.68 26.79) (end 106.68 41.79) (width 0.25) (layer F.Cu) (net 11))
 (segment (start 81.844001 43.274999) (end 87.63 49.060998) (width 0.25) (layer F.Cu) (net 11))
 (segment (start 79.915001 43.274999) (end 81.844001 43.274999) (width 0.25) (layer F.Cu) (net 11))
 (segment (start 78.74 44.45) (end 79.915001 43.274999) (width 0.25) (layer F.Cu) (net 11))
 (segment (start 106.68 43.54) (end 106.68 41.79) (width 0.25) (layer F.Cu) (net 11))
 (segment (start 101.159002 49.060998) (end 106.68 43.54) (width 0.25) (layer F.Cu) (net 11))
 (segment (start 87.63 49.060998) (end 101.159002 49.060998) (width 0.25) (layer F.Cu) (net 11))
 (segment (start 144.78 41.79) (end 144.78 26.79) (width 0.25) (layer F.Cu) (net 12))
 (segment (start 81.28 44.45) (end 87.25499 50.42499) (width 0.25) (layer F.Cu) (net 12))
 (segment (start 144.78 43.54) (end 144.78 41.79) (width 0.25) (layer F.Cu) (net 12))
 (segment (start 137.89501 50.42499) (end 144.78 43.54) (width 0.25) (layer F.Cu) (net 12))
 (segment (start 87.25499 50.42499) (end 137.89501 50.42499) (width 0.25) (layer F.Cu) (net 12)))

